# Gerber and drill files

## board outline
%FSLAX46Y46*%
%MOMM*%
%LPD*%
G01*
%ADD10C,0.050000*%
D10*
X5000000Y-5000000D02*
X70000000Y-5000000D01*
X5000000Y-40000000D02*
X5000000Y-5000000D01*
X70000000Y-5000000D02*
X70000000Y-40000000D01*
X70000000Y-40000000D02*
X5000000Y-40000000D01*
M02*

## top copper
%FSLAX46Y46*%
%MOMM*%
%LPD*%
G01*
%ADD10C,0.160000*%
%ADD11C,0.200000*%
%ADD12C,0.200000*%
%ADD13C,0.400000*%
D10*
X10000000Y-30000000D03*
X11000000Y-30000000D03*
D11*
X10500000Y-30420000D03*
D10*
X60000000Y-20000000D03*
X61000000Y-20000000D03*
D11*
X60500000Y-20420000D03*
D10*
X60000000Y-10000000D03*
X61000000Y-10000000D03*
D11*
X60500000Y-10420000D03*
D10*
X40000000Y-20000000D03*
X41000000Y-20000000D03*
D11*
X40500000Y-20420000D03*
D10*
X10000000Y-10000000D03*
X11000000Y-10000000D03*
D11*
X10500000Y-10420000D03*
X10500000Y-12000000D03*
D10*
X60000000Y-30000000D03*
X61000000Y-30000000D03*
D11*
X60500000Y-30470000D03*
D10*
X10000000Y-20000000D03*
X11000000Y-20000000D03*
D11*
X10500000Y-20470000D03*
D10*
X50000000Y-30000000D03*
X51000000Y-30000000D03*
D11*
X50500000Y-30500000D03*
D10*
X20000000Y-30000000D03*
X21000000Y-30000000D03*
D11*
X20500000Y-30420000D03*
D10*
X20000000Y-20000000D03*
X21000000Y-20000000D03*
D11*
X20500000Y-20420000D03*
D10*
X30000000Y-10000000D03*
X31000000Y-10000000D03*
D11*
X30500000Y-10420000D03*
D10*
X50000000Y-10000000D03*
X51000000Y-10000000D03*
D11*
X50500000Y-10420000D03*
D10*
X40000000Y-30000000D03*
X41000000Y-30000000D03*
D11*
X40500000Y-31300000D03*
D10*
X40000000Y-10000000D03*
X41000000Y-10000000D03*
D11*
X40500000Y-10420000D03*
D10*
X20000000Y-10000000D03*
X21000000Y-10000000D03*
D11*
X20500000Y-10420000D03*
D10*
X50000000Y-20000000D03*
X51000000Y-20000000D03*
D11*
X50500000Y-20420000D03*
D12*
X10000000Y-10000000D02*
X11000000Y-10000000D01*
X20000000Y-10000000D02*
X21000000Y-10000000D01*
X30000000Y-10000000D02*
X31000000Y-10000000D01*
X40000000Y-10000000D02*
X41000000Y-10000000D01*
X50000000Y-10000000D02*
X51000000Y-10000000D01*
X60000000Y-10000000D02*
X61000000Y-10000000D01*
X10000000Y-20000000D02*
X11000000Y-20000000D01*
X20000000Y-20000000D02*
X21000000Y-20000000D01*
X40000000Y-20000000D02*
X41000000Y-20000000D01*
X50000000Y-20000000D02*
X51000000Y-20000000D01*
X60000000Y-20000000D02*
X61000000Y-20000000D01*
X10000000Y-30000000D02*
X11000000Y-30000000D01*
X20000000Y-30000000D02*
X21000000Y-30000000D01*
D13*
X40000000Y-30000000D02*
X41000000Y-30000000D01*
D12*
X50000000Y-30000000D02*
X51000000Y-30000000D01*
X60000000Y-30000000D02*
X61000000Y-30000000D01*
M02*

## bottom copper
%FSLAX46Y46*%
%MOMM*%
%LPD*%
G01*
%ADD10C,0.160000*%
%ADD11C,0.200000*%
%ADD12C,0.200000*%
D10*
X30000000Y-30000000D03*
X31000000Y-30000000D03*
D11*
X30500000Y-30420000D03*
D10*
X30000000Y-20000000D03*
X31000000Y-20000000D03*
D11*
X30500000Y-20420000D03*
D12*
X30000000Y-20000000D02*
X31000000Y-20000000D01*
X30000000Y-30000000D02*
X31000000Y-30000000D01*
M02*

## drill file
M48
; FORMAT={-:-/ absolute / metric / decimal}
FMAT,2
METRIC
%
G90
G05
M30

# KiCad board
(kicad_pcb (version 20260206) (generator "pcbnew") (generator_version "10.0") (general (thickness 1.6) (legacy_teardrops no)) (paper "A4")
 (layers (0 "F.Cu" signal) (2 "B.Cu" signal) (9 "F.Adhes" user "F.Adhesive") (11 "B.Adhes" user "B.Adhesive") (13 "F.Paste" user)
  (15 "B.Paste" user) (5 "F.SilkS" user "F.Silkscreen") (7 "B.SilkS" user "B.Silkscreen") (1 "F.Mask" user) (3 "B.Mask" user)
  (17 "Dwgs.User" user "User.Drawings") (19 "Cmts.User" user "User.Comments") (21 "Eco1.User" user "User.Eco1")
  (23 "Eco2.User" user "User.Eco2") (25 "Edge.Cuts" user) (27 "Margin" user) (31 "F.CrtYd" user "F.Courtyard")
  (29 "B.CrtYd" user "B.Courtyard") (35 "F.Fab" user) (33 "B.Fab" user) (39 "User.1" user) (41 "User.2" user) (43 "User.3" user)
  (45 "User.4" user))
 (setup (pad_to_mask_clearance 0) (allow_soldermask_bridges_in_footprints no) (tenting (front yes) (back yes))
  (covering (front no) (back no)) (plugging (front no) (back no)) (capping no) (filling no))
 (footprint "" (layer "F.Cu") (at 10 30)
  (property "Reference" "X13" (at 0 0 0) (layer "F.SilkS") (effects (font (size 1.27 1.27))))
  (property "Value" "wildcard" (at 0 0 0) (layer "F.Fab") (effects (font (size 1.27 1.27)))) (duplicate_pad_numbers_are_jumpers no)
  (pad "1" smd circle (at 0 0) (size 0.16 0.16) (layers "F.Cu") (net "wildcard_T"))
  (pad "2" smd circle (at 1 0) (size 0.16 0.16) (layers "F.Cu") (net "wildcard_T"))
  (pad "3" smd circle (at 0.5 0.42) (size 0.2 0.2) (layers "F.Cu") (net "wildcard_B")))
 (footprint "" (layer "F.Cu") (at 60 20)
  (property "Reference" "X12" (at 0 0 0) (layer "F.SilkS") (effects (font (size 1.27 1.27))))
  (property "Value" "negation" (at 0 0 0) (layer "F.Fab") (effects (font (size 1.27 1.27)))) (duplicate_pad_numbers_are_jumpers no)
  (pad "1" smd circle (at 0 0) (size 0.16 0.16) (layers "F.Cu") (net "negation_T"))
  (pad "2" smd circle (at 1 0) (size 0.16 0.16) (layers "F.Cu") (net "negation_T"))
  (pad "3" smd circle (at 0.5 0.42) (size 0.2 0.2) (layers "F.Cu") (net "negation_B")))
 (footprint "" (layer "F.Cu") (at 60 10)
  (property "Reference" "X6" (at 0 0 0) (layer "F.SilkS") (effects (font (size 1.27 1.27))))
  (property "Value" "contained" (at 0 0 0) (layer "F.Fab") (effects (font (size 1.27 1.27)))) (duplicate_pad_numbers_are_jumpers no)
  (pad "1" smd circle (at 0 0) (size 0.16 0.16) (layers "F.Cu") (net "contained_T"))
  (pad "2" smd circle (at 1 0) (size 0.16 0.16) (layers "F.Cu") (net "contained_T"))
  (pad "3" smd circle (at 0.5 0.42) (size 0.2 0.2) (layers "F.Cu") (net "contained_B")))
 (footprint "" (layer "F.Cu") (at 40 20)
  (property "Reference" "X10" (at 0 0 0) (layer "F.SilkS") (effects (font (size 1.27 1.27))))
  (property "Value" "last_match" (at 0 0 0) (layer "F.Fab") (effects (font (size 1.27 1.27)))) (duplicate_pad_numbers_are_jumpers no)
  (pad "1" smd circle (at 0 0) (size 0.16 0.16) (layers "F.Cu") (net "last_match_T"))
  (pad "2" smd circle (at 1 0) (size 0.16 0.16) (layers "F.Cu") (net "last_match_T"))
  (pad "3" smd circle (at 0.5 0.42) (size 0.2 0.2) (layers "F.Cu") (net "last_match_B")))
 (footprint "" (layer "F.Cu") (at 10 10)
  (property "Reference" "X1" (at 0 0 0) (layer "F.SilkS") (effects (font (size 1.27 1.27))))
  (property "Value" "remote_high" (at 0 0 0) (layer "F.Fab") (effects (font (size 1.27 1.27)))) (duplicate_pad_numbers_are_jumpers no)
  (pad "1" smd circle (at 0 0) (size 0.16 0.16) (layers "F.Cu") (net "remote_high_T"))
  (pad "2" smd circle (at 1 0) (size 0.16 0.16) (layers "F.Cu") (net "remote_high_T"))
  (pad "3" smd circle (at 0.5 0.42) (size 0.2 0.2) (layers "F.Cu") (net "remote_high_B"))
  (pad "4" smd circle (at 0.5 2) (size 0.2 0.2) (layers "F.Cu") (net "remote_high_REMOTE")))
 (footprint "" (layer "F.Cu") (at 60 30)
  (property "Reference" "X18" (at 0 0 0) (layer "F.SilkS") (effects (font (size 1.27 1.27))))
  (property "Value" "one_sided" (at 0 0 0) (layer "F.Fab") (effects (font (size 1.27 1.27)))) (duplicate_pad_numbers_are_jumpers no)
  (pad "1" smd circle (at 0 0) (size 0.16 0.16) (layers "F.Cu") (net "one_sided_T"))
  (pad "2" smd circle (at 1 0) (size 0.16 0.16) (layers "F.Cu") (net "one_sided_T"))
  (pad "3" smd circle (at 0.5 0.47) (size 0.2 0.2) (layers "F.Cu") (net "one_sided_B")))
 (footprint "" (layer "F.Cu") (at 10 20)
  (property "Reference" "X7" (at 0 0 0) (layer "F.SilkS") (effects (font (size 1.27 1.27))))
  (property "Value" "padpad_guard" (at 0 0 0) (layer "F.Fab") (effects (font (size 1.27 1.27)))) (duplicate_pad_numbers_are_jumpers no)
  (pad "1" smd circle (at 0 0) (size 0.16 0.16) (layers "F.Cu") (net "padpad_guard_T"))
  (pad "2" smd circle (at 1 0) (size 0.16 0.16) (layers "F.Cu") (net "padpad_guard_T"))
  (pad "3" smd circle (at 0.5 0.47) (size 0.2 0.2) (layers "F.Cu") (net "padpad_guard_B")))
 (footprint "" (layer "F.Cu") (at 50 30)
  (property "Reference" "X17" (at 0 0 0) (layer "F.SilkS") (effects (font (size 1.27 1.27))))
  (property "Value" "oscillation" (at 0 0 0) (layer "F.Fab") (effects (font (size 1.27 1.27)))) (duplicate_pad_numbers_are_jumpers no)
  (pad "1" smd circle (at 0 0) (size 0.16 0.16) (layers "F.Cu") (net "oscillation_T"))
  (pad "2" smd circle (at 1 0) (size 0.16 0.16) (layers "F.Cu") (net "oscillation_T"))
  (pad "3" smd circle (at 0.5 0.5) (size 0.2 0.2) (layers "F.Cu") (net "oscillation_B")))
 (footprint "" (layer "F.Cu") (at 20 30)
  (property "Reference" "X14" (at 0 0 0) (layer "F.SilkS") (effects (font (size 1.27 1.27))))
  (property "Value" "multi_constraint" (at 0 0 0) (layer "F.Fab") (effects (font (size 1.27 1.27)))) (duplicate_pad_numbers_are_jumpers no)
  (pad "1" smd circle (at 0 0) (size 0.16 0.16) (layers "F.Cu") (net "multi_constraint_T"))
  (pad "2" smd circle (at 1 0) (size 0.16 0.16) (layers "F.Cu") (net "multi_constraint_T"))
  (pad "3" smd circle (at 0.5 0.42) (size 0.2 0.2) (layers "F.Cu") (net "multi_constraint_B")))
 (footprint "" (layer "F.Cu") (at 30 30)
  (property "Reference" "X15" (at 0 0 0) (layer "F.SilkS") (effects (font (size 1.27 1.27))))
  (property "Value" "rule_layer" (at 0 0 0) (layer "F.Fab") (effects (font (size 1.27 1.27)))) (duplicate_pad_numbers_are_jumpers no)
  (pad "1" smd circle (at 0 0) (size 0.16 0.16) (layers "B.Cu") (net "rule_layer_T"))
  (pad "2" smd circle (at 1 0) (size 0.16 0.16) (layers "B.Cu") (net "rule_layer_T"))
  (pad "3" smd circle (at 0.5 0.42) (size 0.2 0.2) (layers "B.Cu") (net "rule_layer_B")))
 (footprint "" (layer "F.Cu") (at 20 20)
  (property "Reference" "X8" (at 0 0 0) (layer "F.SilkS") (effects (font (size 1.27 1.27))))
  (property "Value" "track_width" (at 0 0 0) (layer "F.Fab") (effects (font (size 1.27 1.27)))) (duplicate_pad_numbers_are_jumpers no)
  (pad "1" smd circle (at 0 0) (size 0.16 0.16) (layers "F.Cu") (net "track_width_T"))
  (pad "2" smd circle (at 1 0) (size 0.16 0.16) (layers "F.Cu") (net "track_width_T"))
  (pad "3" smd circle (at 0.5 0.42) (size 0.2 0.2) (layers "F.Cu") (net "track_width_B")))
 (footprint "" (layer "F.Cu") (at 30 10)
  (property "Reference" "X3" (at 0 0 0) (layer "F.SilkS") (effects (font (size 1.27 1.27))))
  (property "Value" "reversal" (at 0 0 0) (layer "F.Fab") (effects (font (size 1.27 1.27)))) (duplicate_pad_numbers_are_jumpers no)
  (pad "1" smd circle (at 0 0) (size 0.16 0.16) (layers "F.Cu") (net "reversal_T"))
  (pad "2" smd circle (at 1 0) (size 0.16 0.16) (layers "F.Cu") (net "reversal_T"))
  (pad "3" smd circle (at 0.5 0.42) (size 0.2 0.2) (layers "F.Cu") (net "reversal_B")))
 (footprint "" (layer "F.Cu") (at 50 10)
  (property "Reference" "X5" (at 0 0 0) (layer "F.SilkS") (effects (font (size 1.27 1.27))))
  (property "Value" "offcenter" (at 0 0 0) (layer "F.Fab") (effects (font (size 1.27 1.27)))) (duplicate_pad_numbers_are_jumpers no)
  (pad "1" smd circle (at 0 0) (size 0.16 0.16) (layers "F.Cu") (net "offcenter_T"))
  (pad "2" smd circle (at 1 0) (size 0.16 0.16) (layers "F.Cu") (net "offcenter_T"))
  (pad "3" smd circle (at 0.5 0.42) (size 0.2 0.2) (layers "F.Cu") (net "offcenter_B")))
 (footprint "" (layer "F.Cu") (at 40 30)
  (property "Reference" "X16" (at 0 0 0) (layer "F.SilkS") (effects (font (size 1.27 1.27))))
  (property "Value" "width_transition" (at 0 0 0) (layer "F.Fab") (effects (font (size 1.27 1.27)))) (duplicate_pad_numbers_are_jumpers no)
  (pad "1" smd circle (at 0 0) (size 0.16 0.16) (layers "F.Cu") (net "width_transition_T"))
  (pad "2" smd circle (at 1 0) (size 0.16 0.16) (layers "F.Cu") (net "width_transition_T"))
  (pad "3" smd circle (at 0.5 1.3) (size 0.2 0.2) (layers "F.Cu") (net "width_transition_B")))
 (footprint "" (layer "F.Cu") (at 30 20)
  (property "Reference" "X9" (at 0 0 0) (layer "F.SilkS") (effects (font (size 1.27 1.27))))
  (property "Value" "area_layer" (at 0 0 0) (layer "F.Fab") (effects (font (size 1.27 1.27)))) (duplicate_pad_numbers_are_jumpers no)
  (pad "1" smd circle (at 0 0) (size 0.16 0.16) (layers "B.Cu") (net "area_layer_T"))
  (pad "2" smd circle (at 1 0) (size 0.16 0.16) (layers "B.Cu") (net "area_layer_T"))
  (pad "3" smd circle (at 0.5 0.42) (size 0.2 0.2) (layers "B.Cu") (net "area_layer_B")))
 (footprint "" (layer "F.Cu") (at 40 10)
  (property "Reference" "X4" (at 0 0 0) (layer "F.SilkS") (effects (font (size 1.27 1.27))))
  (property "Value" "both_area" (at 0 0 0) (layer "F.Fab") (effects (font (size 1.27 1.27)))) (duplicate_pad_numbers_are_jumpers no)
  (pad "1" smd circle (at 0 0) (size 0.16 0.16) (layers "F.Cu") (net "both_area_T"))
  (pad "2" smd circle (at 1 0) (size 0.16 0.16) (layers "F.Cu") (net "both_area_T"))
  (pad "3" smd circle (at 0.5 0.42) (size 0.2 0.2) (layers "F.Cu") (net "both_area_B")))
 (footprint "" (layer "F.Cu") (at 20 10)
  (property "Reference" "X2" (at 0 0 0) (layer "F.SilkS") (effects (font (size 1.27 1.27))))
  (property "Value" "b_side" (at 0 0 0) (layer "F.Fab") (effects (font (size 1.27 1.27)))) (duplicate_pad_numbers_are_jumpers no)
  (pad "1" smd circle (at 0 0) (size 0.16 0.16) (layers "F.Cu") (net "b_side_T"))
  (pad "2" smd circle (at 1 0) (size 0.16 0.16) (layers "F.Cu") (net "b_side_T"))
  (pad "3" smd circle (at 0.5 0.42) (size 0.2 0.2) (layers "F.Cu") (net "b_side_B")))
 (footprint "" (layer "F.Cu") (at 50 20)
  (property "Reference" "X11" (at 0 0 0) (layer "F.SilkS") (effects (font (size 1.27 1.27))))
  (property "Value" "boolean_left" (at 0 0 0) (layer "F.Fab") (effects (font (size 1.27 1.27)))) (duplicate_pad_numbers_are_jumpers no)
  (pad "1" smd circle (at 0 0) (size 0.16 0.16) (layers "F.Cu") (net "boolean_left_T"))
  (pad "2" smd circle (at 1 0) (size 0.16 0.16) (layers "F.Cu") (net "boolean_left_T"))
  (pad "3" smd circle (at 0.5 0.42) (size 0.2 0.2) (layers "F.Cu") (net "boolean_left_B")))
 (gr_line (start 5 5) (end 70 5) (stroke (width 0.05) (type default)) (layer "Edge.Cuts"))
 (gr_line (start 5 40) (end 5 5) (stroke (width 0.05) (type default)) (layer "Edge.Cuts"))
 (gr_line (start 70 5) (end 70 40) (stroke (width 0.05) (type default)) (layer "Edge.Cuts"))
 (gr_line (start 70 40) (end 5 40) (stroke (width 0.05) (type default)) (layer "Edge.Cuts"))
 (segment (start 10 10) (end 11 10) (width 0.2) (layer "F.Cu") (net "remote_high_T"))
 (segment (start 20 10) (end 21 10) (width 0.2) (layer "F.Cu") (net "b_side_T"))
 (segment (start 30 10) (end 31 10) (width 0.2) (layer "F.Cu") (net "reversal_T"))
 (segment (start 40 10) (end 41 10) (width 0.2) (layer "F.Cu") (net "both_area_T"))
 (segment (start 50 10) (end 51 10) (width 0.2) (layer "F.Cu") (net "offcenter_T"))
 (segment (start 60 10) (end 61 10) (width 0.2) (layer "F.Cu") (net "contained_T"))
 (segment (start 10 20) (end 11 20) (width 0.2) (layer "F.Cu") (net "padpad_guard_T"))
 (segment (start 20 20) (end 21 20) (width 0.2) (layer "F.Cu") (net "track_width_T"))
 (segment (start 30 20) (end 31 20) (width 0.2) (layer "B.Cu") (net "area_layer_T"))
 (segment (start 40 20) (end 41 20) (width 0.2) (layer "F.Cu") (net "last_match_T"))
 (segment (start 50 20) (end 51 20) (width 0.2) (layer "F.Cu") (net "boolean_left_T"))
 (segment (start 60 20) (end 61 20) (width 0.2) (layer "F.Cu") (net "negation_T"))
 (segment (start 10 30) (end 11 30) (width 0.2) (layer "F.Cu") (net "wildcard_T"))
 (segment (start 20 30) (end 21 30) (width 0.2) (layer "F.Cu") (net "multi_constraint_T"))
 (segment (start 30 30) (end 31 30) (width 0.2) (layer "B.Cu") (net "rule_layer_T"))
 (segment (start 40 30) (end 41 30) (width 0.4) (layer "F.Cu") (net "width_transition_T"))
 (segment (start 50 30) (end 51 30) (width 0.2) (layer "F.Cu") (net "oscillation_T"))
 (segment (start 60 30) (end 61 30) (width 0.2) (layer "F.Cu") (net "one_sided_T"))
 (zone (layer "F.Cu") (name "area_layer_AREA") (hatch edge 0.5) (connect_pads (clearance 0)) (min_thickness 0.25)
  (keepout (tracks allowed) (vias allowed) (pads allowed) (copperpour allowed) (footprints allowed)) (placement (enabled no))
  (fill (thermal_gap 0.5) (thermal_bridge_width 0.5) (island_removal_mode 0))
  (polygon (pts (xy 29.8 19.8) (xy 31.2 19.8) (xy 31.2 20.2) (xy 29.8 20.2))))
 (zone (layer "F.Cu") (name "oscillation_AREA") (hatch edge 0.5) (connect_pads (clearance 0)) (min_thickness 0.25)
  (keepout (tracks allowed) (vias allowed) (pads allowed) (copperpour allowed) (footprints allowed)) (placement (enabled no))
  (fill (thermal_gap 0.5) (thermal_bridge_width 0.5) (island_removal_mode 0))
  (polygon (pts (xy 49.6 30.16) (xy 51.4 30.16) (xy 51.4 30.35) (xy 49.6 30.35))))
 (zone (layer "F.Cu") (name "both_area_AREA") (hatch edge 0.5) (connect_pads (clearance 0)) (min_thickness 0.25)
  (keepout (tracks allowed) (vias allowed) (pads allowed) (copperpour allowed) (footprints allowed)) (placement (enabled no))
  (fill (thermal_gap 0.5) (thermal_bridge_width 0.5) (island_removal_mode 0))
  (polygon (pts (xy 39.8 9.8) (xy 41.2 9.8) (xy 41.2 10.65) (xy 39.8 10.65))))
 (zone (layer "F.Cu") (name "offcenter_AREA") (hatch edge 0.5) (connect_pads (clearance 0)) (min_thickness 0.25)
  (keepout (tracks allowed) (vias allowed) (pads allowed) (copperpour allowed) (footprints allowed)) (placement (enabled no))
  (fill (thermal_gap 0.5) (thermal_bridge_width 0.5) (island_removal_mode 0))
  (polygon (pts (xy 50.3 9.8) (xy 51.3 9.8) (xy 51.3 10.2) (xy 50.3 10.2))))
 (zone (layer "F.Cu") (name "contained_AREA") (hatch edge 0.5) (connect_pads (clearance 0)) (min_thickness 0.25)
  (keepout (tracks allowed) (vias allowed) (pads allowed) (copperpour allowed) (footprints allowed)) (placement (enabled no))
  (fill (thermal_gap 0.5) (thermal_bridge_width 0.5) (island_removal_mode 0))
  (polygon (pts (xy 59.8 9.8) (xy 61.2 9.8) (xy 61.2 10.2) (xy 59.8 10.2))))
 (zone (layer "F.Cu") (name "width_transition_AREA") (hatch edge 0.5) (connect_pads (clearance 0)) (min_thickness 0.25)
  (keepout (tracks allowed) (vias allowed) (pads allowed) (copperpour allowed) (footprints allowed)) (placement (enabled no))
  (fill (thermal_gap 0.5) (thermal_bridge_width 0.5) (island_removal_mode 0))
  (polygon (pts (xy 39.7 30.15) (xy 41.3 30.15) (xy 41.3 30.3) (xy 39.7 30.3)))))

